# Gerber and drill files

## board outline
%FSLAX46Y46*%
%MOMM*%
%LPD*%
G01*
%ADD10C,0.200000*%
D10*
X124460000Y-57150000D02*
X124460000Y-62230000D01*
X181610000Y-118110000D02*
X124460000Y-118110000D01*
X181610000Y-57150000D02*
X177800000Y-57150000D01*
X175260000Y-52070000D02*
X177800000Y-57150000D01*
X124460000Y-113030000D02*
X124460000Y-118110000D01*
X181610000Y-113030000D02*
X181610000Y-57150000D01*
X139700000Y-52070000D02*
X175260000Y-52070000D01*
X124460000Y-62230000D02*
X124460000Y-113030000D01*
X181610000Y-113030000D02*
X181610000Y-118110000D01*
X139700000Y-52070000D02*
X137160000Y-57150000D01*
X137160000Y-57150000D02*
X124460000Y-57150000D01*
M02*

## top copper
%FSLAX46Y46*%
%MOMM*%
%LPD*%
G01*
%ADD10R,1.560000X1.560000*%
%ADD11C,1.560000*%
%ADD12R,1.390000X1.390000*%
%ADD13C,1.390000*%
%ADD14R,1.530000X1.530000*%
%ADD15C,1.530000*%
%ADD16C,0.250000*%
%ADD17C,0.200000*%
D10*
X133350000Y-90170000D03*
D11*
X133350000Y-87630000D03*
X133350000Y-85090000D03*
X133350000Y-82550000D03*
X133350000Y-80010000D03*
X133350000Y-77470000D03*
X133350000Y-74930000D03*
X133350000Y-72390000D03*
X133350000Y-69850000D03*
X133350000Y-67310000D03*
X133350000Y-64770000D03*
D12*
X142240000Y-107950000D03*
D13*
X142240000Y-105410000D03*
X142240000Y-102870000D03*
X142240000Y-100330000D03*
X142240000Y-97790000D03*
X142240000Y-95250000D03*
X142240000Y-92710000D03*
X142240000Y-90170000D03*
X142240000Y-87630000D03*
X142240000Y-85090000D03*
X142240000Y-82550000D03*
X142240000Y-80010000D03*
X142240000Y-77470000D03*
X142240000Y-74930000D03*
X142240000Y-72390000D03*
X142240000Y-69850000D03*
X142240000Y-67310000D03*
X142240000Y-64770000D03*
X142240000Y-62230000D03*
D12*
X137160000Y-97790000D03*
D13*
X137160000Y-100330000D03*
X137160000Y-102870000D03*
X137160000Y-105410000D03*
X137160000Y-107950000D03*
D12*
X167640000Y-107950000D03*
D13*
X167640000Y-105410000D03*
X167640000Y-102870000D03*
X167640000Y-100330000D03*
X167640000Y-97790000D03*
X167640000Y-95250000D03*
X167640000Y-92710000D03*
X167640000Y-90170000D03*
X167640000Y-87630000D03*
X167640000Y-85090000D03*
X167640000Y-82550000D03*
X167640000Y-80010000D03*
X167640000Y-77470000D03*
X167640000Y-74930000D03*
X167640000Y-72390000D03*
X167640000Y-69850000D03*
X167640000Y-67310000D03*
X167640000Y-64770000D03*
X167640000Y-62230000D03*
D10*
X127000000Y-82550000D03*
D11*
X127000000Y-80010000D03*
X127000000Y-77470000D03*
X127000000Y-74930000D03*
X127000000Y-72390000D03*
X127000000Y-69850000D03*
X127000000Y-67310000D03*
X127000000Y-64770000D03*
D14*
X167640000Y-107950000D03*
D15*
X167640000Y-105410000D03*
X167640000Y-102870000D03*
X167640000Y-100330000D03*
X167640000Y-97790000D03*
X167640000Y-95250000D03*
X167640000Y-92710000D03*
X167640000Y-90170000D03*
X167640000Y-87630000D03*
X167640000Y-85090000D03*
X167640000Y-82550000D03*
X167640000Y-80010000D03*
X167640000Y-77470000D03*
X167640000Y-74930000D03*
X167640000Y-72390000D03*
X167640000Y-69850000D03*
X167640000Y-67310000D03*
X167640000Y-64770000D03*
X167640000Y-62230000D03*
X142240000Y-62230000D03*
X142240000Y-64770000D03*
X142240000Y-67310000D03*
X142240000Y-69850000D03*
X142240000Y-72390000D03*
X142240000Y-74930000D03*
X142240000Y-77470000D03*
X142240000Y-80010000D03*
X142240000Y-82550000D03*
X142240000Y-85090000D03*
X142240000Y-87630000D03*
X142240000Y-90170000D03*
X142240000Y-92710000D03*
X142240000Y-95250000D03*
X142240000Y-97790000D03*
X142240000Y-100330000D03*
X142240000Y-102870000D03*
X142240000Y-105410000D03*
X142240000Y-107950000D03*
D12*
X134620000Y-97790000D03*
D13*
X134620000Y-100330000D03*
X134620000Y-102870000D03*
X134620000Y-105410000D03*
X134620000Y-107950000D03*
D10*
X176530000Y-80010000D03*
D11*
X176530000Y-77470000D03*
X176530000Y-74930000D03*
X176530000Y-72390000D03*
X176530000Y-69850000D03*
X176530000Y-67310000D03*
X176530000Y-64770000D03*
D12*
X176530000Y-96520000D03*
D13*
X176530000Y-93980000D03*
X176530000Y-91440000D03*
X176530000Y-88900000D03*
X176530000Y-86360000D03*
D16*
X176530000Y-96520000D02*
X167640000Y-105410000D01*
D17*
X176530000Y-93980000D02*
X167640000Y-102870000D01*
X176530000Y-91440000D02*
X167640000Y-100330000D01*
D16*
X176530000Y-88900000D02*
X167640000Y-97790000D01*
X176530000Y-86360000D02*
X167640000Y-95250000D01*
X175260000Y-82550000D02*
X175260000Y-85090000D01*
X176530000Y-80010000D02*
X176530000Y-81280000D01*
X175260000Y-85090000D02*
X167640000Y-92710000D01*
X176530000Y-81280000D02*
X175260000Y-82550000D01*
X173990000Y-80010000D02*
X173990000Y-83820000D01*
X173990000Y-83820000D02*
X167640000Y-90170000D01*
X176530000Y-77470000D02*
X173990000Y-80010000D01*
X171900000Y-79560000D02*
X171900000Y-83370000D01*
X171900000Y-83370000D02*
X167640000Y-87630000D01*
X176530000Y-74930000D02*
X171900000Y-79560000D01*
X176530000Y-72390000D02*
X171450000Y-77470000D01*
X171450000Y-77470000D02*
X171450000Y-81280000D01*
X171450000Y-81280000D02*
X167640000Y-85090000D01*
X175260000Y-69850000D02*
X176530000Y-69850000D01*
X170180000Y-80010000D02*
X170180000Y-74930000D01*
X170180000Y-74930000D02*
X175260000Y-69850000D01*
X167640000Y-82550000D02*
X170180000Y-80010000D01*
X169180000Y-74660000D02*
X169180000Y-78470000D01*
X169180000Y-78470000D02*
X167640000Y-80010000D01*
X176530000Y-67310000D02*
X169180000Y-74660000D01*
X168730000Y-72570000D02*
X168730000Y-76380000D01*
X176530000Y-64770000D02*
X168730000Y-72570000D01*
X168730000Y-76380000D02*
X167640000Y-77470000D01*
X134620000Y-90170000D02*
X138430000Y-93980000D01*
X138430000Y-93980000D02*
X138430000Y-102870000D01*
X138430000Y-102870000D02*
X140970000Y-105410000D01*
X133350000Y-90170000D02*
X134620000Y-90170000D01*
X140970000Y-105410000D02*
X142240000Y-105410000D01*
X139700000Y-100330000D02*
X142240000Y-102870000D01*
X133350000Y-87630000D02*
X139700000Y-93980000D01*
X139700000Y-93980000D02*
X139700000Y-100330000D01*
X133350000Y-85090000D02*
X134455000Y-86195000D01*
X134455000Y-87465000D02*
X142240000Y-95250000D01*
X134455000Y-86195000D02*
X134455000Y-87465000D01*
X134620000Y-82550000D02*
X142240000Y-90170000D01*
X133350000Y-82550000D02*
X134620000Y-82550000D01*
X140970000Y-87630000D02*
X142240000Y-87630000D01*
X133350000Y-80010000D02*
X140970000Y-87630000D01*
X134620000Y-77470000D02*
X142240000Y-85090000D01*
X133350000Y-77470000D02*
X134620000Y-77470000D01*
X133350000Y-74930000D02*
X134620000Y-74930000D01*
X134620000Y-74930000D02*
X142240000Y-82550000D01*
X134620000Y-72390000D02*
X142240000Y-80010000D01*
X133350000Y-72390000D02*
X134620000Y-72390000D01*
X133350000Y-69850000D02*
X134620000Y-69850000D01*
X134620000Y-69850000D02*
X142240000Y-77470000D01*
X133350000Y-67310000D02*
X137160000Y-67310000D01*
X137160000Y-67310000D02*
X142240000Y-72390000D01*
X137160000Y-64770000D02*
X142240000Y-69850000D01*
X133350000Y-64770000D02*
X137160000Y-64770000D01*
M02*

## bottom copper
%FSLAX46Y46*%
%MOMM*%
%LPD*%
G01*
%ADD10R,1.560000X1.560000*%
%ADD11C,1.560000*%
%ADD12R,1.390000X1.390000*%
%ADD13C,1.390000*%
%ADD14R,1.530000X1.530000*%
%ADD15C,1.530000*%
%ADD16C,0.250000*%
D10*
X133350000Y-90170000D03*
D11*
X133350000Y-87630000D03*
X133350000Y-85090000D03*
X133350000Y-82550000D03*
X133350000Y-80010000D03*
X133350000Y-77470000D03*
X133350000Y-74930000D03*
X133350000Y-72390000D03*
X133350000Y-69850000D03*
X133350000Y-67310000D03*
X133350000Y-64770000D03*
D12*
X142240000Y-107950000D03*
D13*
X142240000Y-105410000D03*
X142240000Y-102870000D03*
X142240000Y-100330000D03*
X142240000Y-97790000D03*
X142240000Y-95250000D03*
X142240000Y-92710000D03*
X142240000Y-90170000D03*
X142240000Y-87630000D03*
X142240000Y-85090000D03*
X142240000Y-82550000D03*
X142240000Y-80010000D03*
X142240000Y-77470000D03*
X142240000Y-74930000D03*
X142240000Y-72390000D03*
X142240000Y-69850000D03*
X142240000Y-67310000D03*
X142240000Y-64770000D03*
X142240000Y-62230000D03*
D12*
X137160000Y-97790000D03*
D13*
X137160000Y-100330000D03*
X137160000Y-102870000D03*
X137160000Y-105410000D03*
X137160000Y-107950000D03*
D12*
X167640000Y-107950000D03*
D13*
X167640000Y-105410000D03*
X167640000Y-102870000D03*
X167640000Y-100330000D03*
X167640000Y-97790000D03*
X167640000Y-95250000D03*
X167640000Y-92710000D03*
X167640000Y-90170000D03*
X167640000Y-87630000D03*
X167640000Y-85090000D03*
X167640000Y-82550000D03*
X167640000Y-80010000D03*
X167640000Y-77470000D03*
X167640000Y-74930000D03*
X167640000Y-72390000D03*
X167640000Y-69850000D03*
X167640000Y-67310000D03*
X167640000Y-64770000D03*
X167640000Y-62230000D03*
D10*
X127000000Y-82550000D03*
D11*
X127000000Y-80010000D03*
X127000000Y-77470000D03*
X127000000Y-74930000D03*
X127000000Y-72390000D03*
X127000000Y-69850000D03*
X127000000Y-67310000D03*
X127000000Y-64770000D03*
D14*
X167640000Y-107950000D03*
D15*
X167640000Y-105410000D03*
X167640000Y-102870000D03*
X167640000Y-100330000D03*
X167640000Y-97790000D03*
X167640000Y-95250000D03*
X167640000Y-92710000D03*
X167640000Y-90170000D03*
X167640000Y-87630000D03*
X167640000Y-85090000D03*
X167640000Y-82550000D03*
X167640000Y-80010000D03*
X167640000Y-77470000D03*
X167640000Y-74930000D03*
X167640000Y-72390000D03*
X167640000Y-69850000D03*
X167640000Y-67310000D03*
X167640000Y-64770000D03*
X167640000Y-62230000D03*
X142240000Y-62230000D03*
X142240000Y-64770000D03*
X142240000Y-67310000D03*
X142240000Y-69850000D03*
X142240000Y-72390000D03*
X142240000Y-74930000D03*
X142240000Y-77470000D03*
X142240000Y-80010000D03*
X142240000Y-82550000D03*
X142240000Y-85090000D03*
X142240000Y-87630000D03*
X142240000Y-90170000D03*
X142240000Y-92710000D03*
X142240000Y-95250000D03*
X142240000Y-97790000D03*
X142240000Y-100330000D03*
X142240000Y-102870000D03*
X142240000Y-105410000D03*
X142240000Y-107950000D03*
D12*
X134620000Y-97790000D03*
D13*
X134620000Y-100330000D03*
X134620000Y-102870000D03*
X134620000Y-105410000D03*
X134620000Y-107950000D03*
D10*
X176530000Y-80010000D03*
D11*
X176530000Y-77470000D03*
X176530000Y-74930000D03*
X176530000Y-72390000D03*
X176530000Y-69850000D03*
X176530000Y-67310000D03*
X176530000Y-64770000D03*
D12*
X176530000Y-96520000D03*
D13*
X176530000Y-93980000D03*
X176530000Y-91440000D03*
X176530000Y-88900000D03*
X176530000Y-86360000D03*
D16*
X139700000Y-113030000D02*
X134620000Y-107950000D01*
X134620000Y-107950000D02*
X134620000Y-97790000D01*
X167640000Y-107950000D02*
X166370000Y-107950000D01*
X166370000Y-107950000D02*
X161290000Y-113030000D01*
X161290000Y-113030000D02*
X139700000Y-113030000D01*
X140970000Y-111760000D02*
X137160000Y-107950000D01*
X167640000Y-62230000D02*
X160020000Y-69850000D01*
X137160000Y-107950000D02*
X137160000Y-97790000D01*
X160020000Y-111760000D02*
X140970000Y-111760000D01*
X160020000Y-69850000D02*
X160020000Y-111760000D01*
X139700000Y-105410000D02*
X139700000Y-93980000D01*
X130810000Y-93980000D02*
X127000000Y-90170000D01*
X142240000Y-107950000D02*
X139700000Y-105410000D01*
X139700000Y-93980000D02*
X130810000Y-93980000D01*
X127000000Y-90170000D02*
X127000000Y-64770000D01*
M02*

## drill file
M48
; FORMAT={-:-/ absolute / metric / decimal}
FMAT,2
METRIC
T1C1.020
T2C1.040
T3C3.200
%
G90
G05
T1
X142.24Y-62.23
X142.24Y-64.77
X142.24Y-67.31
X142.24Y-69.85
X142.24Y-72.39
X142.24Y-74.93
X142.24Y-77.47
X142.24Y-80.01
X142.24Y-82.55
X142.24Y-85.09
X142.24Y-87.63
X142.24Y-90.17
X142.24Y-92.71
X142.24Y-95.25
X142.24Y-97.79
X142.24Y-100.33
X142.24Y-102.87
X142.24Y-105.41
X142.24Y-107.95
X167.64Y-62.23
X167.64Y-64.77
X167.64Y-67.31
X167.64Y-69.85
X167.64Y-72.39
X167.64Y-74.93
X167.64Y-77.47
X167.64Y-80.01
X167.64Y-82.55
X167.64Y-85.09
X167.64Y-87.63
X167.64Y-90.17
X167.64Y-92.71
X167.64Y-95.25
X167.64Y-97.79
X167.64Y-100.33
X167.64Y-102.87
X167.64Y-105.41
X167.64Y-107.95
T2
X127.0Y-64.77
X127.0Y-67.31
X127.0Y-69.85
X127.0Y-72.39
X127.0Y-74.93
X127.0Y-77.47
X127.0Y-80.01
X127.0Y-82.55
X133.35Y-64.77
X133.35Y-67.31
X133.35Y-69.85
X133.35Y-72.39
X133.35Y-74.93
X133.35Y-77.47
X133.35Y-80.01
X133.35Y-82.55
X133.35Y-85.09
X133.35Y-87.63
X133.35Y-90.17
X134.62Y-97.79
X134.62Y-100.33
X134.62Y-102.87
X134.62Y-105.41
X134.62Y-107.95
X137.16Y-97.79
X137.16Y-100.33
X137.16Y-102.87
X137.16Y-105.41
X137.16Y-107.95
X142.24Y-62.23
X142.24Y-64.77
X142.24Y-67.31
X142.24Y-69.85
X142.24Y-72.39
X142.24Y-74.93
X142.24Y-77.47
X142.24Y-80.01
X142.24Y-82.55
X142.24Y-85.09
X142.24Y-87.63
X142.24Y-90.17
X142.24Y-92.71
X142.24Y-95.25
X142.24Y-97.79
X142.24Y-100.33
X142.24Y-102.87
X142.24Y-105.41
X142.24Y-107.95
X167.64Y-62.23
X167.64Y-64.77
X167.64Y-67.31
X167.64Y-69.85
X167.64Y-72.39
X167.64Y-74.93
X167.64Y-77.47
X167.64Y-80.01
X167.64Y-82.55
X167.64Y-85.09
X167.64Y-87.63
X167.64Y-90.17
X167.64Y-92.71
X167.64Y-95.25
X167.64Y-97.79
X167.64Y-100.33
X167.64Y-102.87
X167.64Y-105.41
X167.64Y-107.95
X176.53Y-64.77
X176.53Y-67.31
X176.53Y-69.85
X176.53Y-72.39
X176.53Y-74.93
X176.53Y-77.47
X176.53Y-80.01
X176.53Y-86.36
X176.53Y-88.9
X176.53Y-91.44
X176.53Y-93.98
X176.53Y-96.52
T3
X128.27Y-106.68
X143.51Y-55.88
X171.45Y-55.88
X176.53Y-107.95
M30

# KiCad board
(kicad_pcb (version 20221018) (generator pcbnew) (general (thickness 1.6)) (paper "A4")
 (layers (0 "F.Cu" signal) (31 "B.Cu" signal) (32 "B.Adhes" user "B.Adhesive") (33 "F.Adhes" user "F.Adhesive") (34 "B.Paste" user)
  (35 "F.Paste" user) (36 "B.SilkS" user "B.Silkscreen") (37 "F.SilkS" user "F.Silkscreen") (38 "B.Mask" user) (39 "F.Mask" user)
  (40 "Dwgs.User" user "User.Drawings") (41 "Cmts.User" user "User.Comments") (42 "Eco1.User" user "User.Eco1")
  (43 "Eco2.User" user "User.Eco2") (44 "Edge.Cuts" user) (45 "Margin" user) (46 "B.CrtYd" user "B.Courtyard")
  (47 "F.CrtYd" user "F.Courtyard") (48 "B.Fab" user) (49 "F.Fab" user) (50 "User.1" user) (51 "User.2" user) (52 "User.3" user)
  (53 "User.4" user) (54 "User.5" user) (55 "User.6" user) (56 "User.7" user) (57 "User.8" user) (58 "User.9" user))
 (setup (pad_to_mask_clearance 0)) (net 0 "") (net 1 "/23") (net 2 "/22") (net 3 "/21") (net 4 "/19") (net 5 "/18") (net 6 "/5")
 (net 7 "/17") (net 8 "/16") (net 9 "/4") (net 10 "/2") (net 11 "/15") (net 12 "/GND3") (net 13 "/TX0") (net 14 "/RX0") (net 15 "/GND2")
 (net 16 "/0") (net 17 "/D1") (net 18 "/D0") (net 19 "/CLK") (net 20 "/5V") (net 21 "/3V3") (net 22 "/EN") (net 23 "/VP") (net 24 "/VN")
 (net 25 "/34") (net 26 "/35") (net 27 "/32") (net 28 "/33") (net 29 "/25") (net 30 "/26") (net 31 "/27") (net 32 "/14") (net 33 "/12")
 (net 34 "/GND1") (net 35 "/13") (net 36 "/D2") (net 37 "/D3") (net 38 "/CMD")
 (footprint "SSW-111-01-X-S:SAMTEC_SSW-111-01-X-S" (layer "F.Cu") (at 133.35 77.47 90)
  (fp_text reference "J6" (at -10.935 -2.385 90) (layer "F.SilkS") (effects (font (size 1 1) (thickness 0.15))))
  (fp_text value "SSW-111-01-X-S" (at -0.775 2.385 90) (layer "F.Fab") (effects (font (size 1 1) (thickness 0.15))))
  (pad "01" thru_hole rect (at -12.7 0 90) (size 1.56 1.56) (drill 1.04) (layers "*.Cu" "*.Mask") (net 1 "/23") (solder_mask_margin 0.102))
  (pad "02" thru_hole circle (at -10.16 0 90) (size 1.56 1.56) (drill 1.04) (layers "*.Cu" "*.Mask") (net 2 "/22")
   (solder_mask_margin 0.102))
  (pad "03" thru_hole circle (at -7.62 0 90) (size 1.56 1.56) (drill 1.04) (layers "*.Cu" "*.Mask") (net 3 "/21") (solder_mask_margin 0.102))
  (pad "04" thru_hole circle (at -5.08 0 90) (size 1.56 1.56) (drill 1.04) (layers "*.Cu" "*.Mask") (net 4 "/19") (solder_mask_margin 0.102))
  (pad "05" thru_hole circle (at -2.54 0 90) (size 1.56 1.56) (drill 1.04) (layers "*.Cu" "*.Mask") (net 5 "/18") (solder_mask_margin 0.102))
  (pad "06" thru_hole circle (at 0 0 90) (size 1.56 1.56) (drill 1.04) (layers "*.Cu" "*.Mask") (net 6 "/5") (solder_mask_margin 0.102))
  (pad "07" thru_hole circle (at 2.54 0 90) (size 1.56 1.56) (drill 1.04) (layers "*.Cu" "*.Mask") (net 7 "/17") (solder_mask_margin 0.102))
  (pad "08" thru_hole circle (at 5.08 0 90) (size 1.56 1.56) (drill 1.04) (layers "*.Cu" "*.Mask") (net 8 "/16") (solder_mask_margin 0.102))
  (pad "09" thru_hole circle (at 7.62 0 90) (size 1.56 1.56) (drill 1.04) (layers "*.Cu" "*.Mask") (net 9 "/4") (solder_mask_margin 0.102))
  (pad "10" thru_hole circle (at 10.16 0 90) (size 1.56 1.56) (drill 1.04) (layers "*.Cu" "*.Mask") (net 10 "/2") (solder_mask_margin 0.102))
  (pad "11" thru_hole circle (at 12.7 0 90) (size 1.56 1.56) (drill 1.04) (layers "*.Cu" "*.Mask") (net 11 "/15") (solder_mask_margin 0.102)))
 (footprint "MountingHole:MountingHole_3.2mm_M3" (layer "F.Cu") (at 128.27 106.68 180)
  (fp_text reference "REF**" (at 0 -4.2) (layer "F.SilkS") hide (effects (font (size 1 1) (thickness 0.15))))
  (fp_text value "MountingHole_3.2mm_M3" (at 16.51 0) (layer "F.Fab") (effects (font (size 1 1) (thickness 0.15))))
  (pad "" np_thru_hole circle (at 0 0 180) (size 3.2 3.2) (drill 3.2) (layers "F&B.Cu" "*.Mask")))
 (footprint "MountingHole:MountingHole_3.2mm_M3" (layer "F.Cu") (at 143.51 55.88 180)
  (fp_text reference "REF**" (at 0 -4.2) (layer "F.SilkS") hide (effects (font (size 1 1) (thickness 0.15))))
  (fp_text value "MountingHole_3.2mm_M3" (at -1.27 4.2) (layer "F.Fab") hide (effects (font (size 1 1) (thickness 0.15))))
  (pad "" np_thru_hole circle (at 0 0 180) (size 3.2 3.2) (drill 3.2) (layers "F&B.Cu" "*.Mask")))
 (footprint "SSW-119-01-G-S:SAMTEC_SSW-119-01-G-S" (layer "F.Cu") (at 142.24 107.95 90)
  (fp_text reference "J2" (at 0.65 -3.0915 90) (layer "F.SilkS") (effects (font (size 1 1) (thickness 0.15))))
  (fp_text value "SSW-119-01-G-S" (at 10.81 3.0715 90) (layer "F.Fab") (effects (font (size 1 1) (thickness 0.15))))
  (pad "01" thru_hole rect (at 0 0 90) (size 1.39 1.39) (drill 1.04) (layers "*.Cu" "*.Mask") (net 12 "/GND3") (solder_mask_margin 0.102))
  (pad "02" thru_hole circle (at 2.54 0 90) (size 1.39 1.39) (drill 1.04) (layers "*.Cu" "*.Mask") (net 1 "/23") (solder_mask_margin 0.102))
  (pad "03" thru_hole circle (at 5.08 0 90) (size 1.39 1.39) (drill 1.04) (layers "*.Cu" "*.Mask") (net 2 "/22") (solder_mask_margin 0.102))
  (pad "04" thru_hole circle (at 7.62 0 90) (size 1.39 1.39) (drill 1.04) (layers "*.Cu" "*.Mask") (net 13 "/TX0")
   (solder_mask_margin 0.102))
  (pad "05" thru_hole circle (at 10.16 0 90) (size 1.39 1.39) (drill 1.04) (layers "*.Cu" "*.Mask") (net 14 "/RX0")
   (solder_mask_margin 0.102))
  (pad "06" thru_hole circle (at 12.7 0 90) (size 1.39 1.39) (drill 1.04) (layers "*.Cu" "*.Mask") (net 3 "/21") (solder_mask_margin 0.102))
  (pad "07" thru_hole circle (at 15.24 0 90) (size 1.39 1.39) (drill 1.04) (layers "*.Cu" "*.Mask") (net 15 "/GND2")
   (solder_mask_margin 0.102))
  (pad "08" thru_hole circle (at 17.78 0 90) (size 1.39 1.39) (drill 1.04) (layers "*.Cu" "*.Mask") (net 4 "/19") (solder_mask_margin 0.102))
  (pad "09" thru_hole circle (at 20.32 0 90) (size 1.39 1.39) (drill 1.04) (layers "*.Cu" "*.Mask") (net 5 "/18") (solder_mask_margin 0.102))
  (pad "10" thru_hole circle (at 22.86 0 90) (size 1.39 1.39) (drill 1.04) (layers "*.Cu" "*.Mask") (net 6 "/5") (solder_mask_margin 0.102))
  (pad "11" thru_hole circle (at 25.4 0 90) (size 1.39 1.39) (drill 1.04) (layers "*.Cu" "*.Mask") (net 7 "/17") (solder_mask_margin 0.102))
  (pad "12" thru_hole circle (at 27.94 0 90) (size 1.39 1.39) (drill 1.04) (layers "*.Cu" "*.Mask") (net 8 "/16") (solder_mask_margin 0.102))
  (pad "13" thru_hole circle (at 30.48 0 90) (size 1.39 1.39) (drill 1.04) (layers "*.Cu" "*.Mask") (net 9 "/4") (solder_mask_margin 0.102))
  (pad "14" thru_hole circle (at 33.02 0 90) (size 1.39 1.39) (drill 1.04) (layers "*.Cu" "*.Mask") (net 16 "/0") (solder_mask_margin 0.102))
  (pad "15" thru_hole circle (at 35.56 0 90) (size 1.39 1.39) (drill 1.04) (layers "*.Cu" "*.Mask") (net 10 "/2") (solder_mask_margin 0.102))
  (pad "16" thru_hole circle (at 38.1 0 90) (size 1.39 1.39) (drill 1.04) (layers "*.Cu" "*.Mask") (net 11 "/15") (solder_mask_margin 0.102))
  (pad "17" thru_hole circle (at 40.64 0 90) (size 1.39 1.39) (drill 1.04) (layers "*.Cu" "*.Mask") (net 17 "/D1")
   (solder_mask_margin 0.102))
  (pad "18" thru_hole circle (at 43.18 0 90) (size 1.39 1.39) (drill 1.04) (layers "*.Cu" "*.Mask") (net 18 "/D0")
   (solder_mask_margin 0.102))
  (pad "19" thru_hole circle (at 45.72 0 90) (size 1.39 1.39) (drill 1.04) (layers "*.Cu" "*.Mask") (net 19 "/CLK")
   (solder_mask_margin 0.102)))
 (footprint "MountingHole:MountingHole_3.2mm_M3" (layer "F.Cu") (at 171.45 55.88 180)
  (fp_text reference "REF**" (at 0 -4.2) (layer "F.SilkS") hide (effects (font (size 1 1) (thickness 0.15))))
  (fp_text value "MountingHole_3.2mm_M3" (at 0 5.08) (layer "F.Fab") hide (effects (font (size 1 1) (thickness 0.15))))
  (pad "" np_thru_hole circle (at 0 0 180) (size 3.2 3.2) (drill 3.2) (layers "F&B.Cu" "*.Mask")))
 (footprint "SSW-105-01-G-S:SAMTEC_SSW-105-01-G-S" (layer "F.Cu") (at 137.16 97.79 -90)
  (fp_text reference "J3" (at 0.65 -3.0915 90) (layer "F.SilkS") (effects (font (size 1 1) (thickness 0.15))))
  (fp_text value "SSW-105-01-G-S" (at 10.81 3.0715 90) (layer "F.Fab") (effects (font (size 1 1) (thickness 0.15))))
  (pad "01" thru_hole rect (at 0 0 270) (size 1.39 1.39) (drill 1.04) (layers "*.Cu" "*.Mask") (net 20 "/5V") (solder_mask_margin 0.102))
  (pad "02" thru_hole circle (at 2.54 0 270) (size 1.39 1.39) (drill 1.04) (layers "*.Cu" "*.Mask") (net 20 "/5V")
   (solder_mask_margin 0.102))
  (pad "03" thru_hole circle (at 5.08 0 270) (size 1.39 1.39) (drill 1.04) (layers "*.Cu" "*.Mask") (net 20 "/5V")
   (solder_mask_margin 0.102))
  (pad "04" thru_hole circle (at 7.62 0 270) (size 1.39 1.39) (drill 1.04) (layers "*.Cu" "*.Mask") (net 20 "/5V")
   (solder_mask_margin 0.102))
  (pad "05" thru_hole circle (at 10.16 0 270) (size 1.39 1.39) (drill 1.04) (layers "*.Cu" "*.Mask") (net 20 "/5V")
   (solder_mask_margin 0.102)))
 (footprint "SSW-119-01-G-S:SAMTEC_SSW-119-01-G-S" (layer "F.Cu") (at 167.64 107.95 90)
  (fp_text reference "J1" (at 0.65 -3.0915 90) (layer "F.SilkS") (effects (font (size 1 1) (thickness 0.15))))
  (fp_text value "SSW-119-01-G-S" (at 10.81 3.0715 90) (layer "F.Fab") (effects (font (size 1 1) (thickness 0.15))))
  (pad "01" thru_hole rect (at 0 0 90) (size 1.39 1.39) (drill 1.04) (layers "*.Cu" "*.Mask") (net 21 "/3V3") (solder_mask_margin 0.102))
  (pad "02" thru_hole circle (at 2.54 0 90) (size 1.39 1.39) (drill 1.04) (layers "*.Cu" "*.Mask") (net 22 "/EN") (solder_mask_margin 0.102))
  (pad "03" thru_hole circle (at 5.08 0 90) (size 1.39 1.39) (drill 1.04) (layers "*.Cu" "*.Mask") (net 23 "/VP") (solder_mask_margin 0.102))
  (pad "04" thru_hole circle (at 7.62 0 90) (size 1.39 1.39) (drill 1.04) (layers "*.Cu" "*.Mask") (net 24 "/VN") (solder_mask_margin 0.102))
  (pad "05" thru_hole circle (at 10.16 0 90) (size 1.39 1.39) (drill 1.04) (layers "*.Cu" "*.Mask") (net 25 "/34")
   (solder_mask_margin 0.102))
  (pad "06" thru_hole circle (at 12.7 0 90) (size 1.39 1.39) (drill 1.04) (layers "*.Cu" "*.Mask") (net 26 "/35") (solder_mask_margin 0.102))
  (pad "07" thru_hole circle (at 15.24 0 90) (size 1.39 1.39) (drill 1.04) (layers "*.Cu" "*.Mask") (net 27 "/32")
   (solder_mask_margin 0.102))
  (pad "08" thru_hole circle (at 17.78 0 90) (size 1.39 1.39) (drill 1.04) (layers "*.Cu" "*.Mask") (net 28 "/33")
   (solder_mask_margin 0.102))
  (pad "09" thru_hole circle (at 20.32 0 90) (size 1.39 1.39) (drill 1.04) (layers "*.Cu" "*.Mask") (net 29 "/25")
   (solder_mask_margin 0.102))
  (pad "10" thru_hole circle (at 22.86 0 90) (size 1.39 1.39) (drill 1.04) (layers "*.Cu" "*.Mask") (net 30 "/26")
   (solder_mask_margin 0.102))
  (pad "11" thru_hole circle (at 25.4 0 90) (size 1.39 1.39) (drill 1.04) (layers "*.Cu" "*.Mask") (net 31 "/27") (solder_mask_margin 0.102))
  (pad "12" thru_hole circle (at 27.94 0 90) (size 1.39 1.39) (drill 1.04) (layers "*.Cu" "*.Mask") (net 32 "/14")
   (solder_mask_margin 0.102))
  (pad "13" thru_hole circle (at 30.48 0 90) (size 1.39 1.39) (drill 1.04) (layers "*.Cu" "*.Mask") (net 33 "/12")
   (solder_mask_margin 0.102))
  (pad "14" thru_hole circle (at 33.02 0 90) (size 1.39 1.39) (drill 1.04) (layers "*.Cu" "*.Mask") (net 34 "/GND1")
   (solder_mask_margin 0.102))
  (pad "15" thru_hole circle (at 35.56 0 90) (size 1.39 1.39) (drill 1.04) (layers "*.Cu" "*.Mask") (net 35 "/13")
   (solder_mask_margin 0.102))
  (pad "16" thru_hole circle (at 38.1 0 90) (size 1.39 1.39) (drill 1.04) (layers "*.Cu" "*.Mask") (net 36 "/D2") (solder_mask_margin 0.102))
  (pad "17" thru_hole circle (at 40.64 0 90) (size 1.39 1.39) (drill 1.04) (layers "*.Cu" "*.Mask") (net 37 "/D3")
   (solder_mask_margin 0.102))
  (pad "18" thru_hole circle (at 43.18 0 90) (size 1.39 1.39) (drill 1.04) (layers "*.Cu" "*.Mask") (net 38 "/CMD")
   (solder_mask_margin 0.102))
  (pad "19" thru_hole circle (at 45.72 0 90) (size 1.39 1.39) (drill 1.04) (layers "*.Cu" "*.Mask") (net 20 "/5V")
   (solder_mask_margin 0.102)))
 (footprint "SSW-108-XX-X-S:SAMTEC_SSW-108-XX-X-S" (layer "F.Cu") (at 127 73.66 90)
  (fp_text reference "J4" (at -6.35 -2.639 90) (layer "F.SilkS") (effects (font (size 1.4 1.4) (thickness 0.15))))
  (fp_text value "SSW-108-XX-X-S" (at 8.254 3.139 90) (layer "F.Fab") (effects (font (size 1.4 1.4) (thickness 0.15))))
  (pad "01" thru_hole rect (at -8.89 0 90) (size 1.56 1.56) (drill 1.04) (layers "*.Cu" "*.Mask") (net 12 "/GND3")
   (solder_mask_margin 0.102))
  (pad "02" thru_hole circle (at -6.35 0 90) (size 1.56 1.56) (drill 1.04) (layers "*.Cu" "*.Mask") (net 12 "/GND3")
   (solder_mask_margin 0.102))
  (pad "03" thru_hole circle (at -3.81 0 90) (size 1.56 1.56) (drill 1.04) (layers "*.Cu" "*.Mask") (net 12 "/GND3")
   (solder_mask_margin 0.102))
  (pad "04" thru_hole circle (at -1.27 0 90) (size 1.56 1.56) (drill 1.04) (layers "*.Cu" "*.Mask") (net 12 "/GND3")
   (solder_mask_margin 0.102))
  (pad "05" thru_hole circle (at 1.27 0 90) (size 1.56 1.56) (drill 1.04) (layers "*.Cu" "*.Mask") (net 12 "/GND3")
   (solder_mask_margin 0.102))
  (pad "06" thru_hole circle (at 3.81 0 90) (size 1.56 1.56) (drill 1.04) (layers "*.Cu" "*.Mask") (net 12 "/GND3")
   (solder_mask_margin 0.102))
  (pad "07" thru_hole circle (at 6.35 0 90) (size 1.56 1.56) (drill 1.04) (layers "*.Cu" "*.Mask") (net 12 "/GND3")
   (solder_mask_margin 0.102))
  (pad "08" thru_hole circle (at 8.89 0 90) (size 1.56 1.56) (drill 1.04) (layers "*.Cu" "*.Mask") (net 12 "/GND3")
   (solder_mask_margin 0.102)))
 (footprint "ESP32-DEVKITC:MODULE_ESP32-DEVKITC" (layer "F.Cu") (at 154.94 85.1 180)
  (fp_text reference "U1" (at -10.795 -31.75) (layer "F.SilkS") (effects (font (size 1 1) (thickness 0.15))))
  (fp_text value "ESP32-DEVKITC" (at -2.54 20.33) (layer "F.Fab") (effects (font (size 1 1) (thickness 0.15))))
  (pad "1" thru_hole rect (at -12.7 -22.85 180) (size 1.53 1.53) (drill 1.02) (layers "*.Cu" "*.Mask") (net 21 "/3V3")
   (solder_mask_margin 0.102))
  (pad "2" thru_hole circle (at -12.7 -20.31 180) (size 1.53 1.53) (drill 1.02) (layers "*.Cu" "*.Mask") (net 22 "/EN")
   (solder_mask_margin 0.102))
  (pad "3" thru_hole circle (at -12.7 -17.77 180) (size 1.53 1.53) (drill 1.02) (layers "*.Cu" "*.Mask") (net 23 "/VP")
   (solder_mask_margin 0.102))
  (pad "4" thru_hole circle (at -12.7 -15.23 180) (size 1.53 1.53) (drill 1.02) (layers "*.Cu" "*.Mask") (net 24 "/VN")
   (solder_mask_margin 0.102))
  (pad "5" thru_hole circle (at -12.7 -12.69 180) (size 1.53 1.53) (drill 1.02) (layers "*.Cu" "*.Mask") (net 25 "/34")
   (solder_mask_margin 0.102))
  (pad "6" thru_hole circle (at -12.7 -10.15 180) (size 1.53 1.53) (drill 1.02) (layers "*.Cu" "*.Mask") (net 26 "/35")
   (solder_mask_margin 0.102))
  (pad "7" thru_hole circle (at -12.7 -7.61 180) (size 1.53 1.53) (drill 1.02) (layers "*.Cu" "*.Mask") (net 27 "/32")
   (solder_mask_margin 0.102))
  (pad "8" thru_hole circle (at -12.7 -5.07 180) (size 1.53 1.53) (drill 1.02) (layers "*.Cu" "*.Mask") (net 28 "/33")
   (solder_mask_margin 0.102))
  (pad "9" thru_hole circle (at -12.7 -2.53 180) (size 1.53 1.53) (drill 1.02) (layers "*.Cu" "*.Mask") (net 29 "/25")
   (solder_mask_margin 0.102))
  (pad "10" thru_hole circle (at -12.7 0.01 180) (size 1.53 1.53) (drill 1.02) (layers "*.Cu" "*.Mask") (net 30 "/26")
   (solder_mask_margin 0.102))
  (pad "11" thru_hole circle (at -12.7 2.55 180) (size 1.53 1.53) (drill 1.02) (layers "*.Cu" "*.Mask") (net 31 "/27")
   (solder_mask_margin 0.102))
  (pad "12" thru_hole circle (at -12.7 5.09 180) (size 1.53 1.53) (drill 1.02) (layers "*.Cu" "*.Mask") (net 32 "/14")
   (solder_mask_margin 0.102))
  (pad "13" thru_hole circle (at -12.7 7.63 180) (size 1.53 1.53) (drill 1.02) (layers "*.Cu" "*.Mask") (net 33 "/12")
   (solder_mask_margin 0.102))
  (pad "14" thru_hole circle (at -12.7 10.17 180) (size 1.53 1.53) (drill 1.02) (layers "*.Cu" "*.Mask") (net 34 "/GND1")
   (solder_mask_margin 0.102))
  (pad "15" thru_hole circle (at -12.7 12.71 180) (size 1.53 1.53) (drill 1.02) (layers "*.Cu" "*.Mask") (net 35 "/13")
   (solder_mask_margin 0.102))
  (pad "16" thru_hole circle (at -12.7 15.25 180) (size 1.53 1.53) (drill 1.02) (layers "*.Cu" "*.Mask") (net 36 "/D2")
   (solder_mask_margin 0.102))
  (pad "17" thru_hole circle (at -12.7 17.79 180) (size 1.53 1.53) (drill 1.02) (layers "*.Cu" "*.Mask") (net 37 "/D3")
   (solder_mask_margin 0.102))
  (pad "18" thru_hole circle (at -12.7 20.33 180) (size 1.53 1.53) (drill 1.02) (layers "*.Cu" "*.Mask") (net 38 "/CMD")
   (solder_mask_margin 0.102))
  (pad "19" thru_hole circle (at -12.7 22.87 180) (size 1.53 1.53) (drill 1.02) (layers "*.Cu" "*.Mask") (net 20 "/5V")
   (solder_mask_margin 0.102))
  (pad "20" thru_hole circle (at 12.7 22.87 180) (size 1.53 1.53) (drill 1.02) (layers "*.Cu" "*.Mask") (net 19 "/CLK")
   (solder_mask_margin 0.102))
  (pad "21" thru_hole circle (at 12.7 20.33 180) (size 1.53 1.53) (drill 1.02) (layers "*.Cu" "*.Mask") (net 18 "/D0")
   (solder_mask_margin 0.102))
  (pad "22" thru_hole circle (at 12.7 17.79 180) (size 1.53 1.53) (drill 1.02) (layers "*.Cu" "*.Mask") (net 17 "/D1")
   (solder_mask_margin 0.102))
  (pad "23" thru_hole circle (at 12.7 15.25 180) (size 1.53 1.53) (drill 1.02) (layers "*.Cu" "*.Mask") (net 11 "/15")
   (solder_mask_margin 0.102))
  (pad "24" thru_hole circle (at 12.7 12.71 180) (size 1.53 1.53) (drill 1.02) (layers "*.Cu" "*.Mask") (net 10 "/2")
   (solder_mask_margin 0.102))
  (pad "25" thru_hole circle (at 12.7 10.17 180) (size 1.53 1.53) (drill 1.02) (layers "*.Cu" "*.Mask") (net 16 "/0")
   (solder_mask_margin 0.102))
  (pad "26" thru_hole circle (at 12.7 7.63 180) (size 1.53 1.53) (drill 1.02) (layers "*.Cu" "*.Mask") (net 9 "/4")
   (solder_mask_margin 0.102))
  (pad "27" thru_hole circle (at 12.7 5.09 180) (size 1.53 1.53) (drill 1.02) (layers "*.Cu" "*.Mask") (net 8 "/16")
   (solder_mask_margin 0.102))
  (pad "28" thru_hole circle (at 12.7 2.55 180) (size 1.53 1.53) (drill 1.02) (layers "*.Cu" "*.Mask") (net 7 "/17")
   (solder_mask_margin 0.102))
  (pad "29" thru_hole circle (at 12.7 0.01 180) (size 1.53 1.53) (drill 1.02) (layers "*.Cu" "*.Mask") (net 6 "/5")
   (solder_mask_margin 0.102))
  (pad "30" thru_hole circle (at 12.7 -2.53 180) (size 1.53 1.53) (drill 1.02) (layers "*.Cu" "*.Mask") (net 5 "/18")
   (solder_mask_margin 0.102))
  (pad "31" thru_hole circle (at 12.7 -5.07 180) (size 1.53 1.53) (drill 1.02) (layers "*.Cu" "*.Mask") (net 4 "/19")
   (solder_mask_margin 0.102))
  (pad "32" thru_hole circle (at 12.7 -7.61 180) (size 1.53 1.53) (drill 1.02) (layers "*.Cu" "*.Mask") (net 15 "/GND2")
   (solder_mask_margin 0.102))
  (pad "33" thru_hole circle (at 12.7 -10.15 180) (size 1.53 1.53) (drill 1.02) (layers "*.Cu" "*.Mask") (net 3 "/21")
   (solder_mask_margin 0.102))
  (pad "34" thru_hole circle (at 12.7 -12.69 180) (size 1.53 1.53) (drill 1.02) (layers "*.Cu" "*.Mask") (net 14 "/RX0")
   (solder_mask_margin 0.102))
  (pad "35" thru_hole circle (at 12.7 -15.23 180) (size 1.53 1.53) (drill 1.02) (layers "*.Cu" "*.Mask") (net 13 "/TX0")
   (solder_mask_margin 0.102))
  (pad "36" thru_hole circle (at 12.7 -17.77 180) (size 1.53 1.53) (drill 1.02) (layers "*.Cu" "*.Mask") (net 2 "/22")
   (solder_mask_margin 0.102))
  (pad "37" thru_hole circle (at 12.7 -20.31 180) (size 1.53 1.53) (drill 1.02) (layers "*.Cu" "*.Mask") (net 1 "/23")
   (solder_mask_margin 0.102))
  (pad "38" thru_hole circle (at 12.7 -22.85 180) (size 1.53 1.53) (drill 1.02) (layers "*.Cu" "*.Mask") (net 12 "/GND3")
   (solder_mask_margin 0.102)))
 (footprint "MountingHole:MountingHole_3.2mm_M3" (layer "F.Cu") (at 176.53 107.95 180)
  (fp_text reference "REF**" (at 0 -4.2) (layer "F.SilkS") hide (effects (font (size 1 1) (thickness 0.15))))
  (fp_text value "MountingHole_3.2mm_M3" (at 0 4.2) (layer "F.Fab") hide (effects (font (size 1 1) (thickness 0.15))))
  (pad "" np_thru_hole circle (at 0 0 180) (size 3.2 3.2) (drill 3.2) (layers "F&B.Cu" "*.Mask")))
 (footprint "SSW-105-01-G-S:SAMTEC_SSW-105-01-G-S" (layer "F.Cu") (at 134.62 97.79 -90)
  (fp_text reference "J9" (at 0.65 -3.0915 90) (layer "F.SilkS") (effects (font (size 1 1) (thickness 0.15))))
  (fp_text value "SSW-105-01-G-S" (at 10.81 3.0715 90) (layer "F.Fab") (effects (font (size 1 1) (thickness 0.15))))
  (pad "01" thru_hole rect (at 0 0 270) (size 1.39 1.39) (drill 1.04) (layers "*.Cu" "*.Mask") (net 21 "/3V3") (solder_mask_margin 0.102))
  (pad "02" thru_hole circle (at 2.54 0 270) (size 1.39 1.39) (drill 1.04) (layers "*.Cu" "*.Mask") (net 21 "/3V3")
   (solder_mask_margin 0.102))
  (pad "03" thru_hole circle (at 5.08 0 270) (size 1.39 1.39) (drill 1.04) (layers "*.Cu" "*.Mask") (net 21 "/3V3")
   (solder_mask_margin 0.102))
  (pad "04" thru_hole circle (at 7.62 0 270) (size 1.39 1.39) (drill 1.04) (layers "*.Cu" "*.Mask") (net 21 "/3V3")
   (solder_mask_margin 0.102))
  (pad "05" thru_hole circle (at 10.16 0 270) (size 1.39 1.39) (drill 1.04) (layers "*.Cu" "*.Mask") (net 21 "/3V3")
   (solder_mask_margin 0.102)))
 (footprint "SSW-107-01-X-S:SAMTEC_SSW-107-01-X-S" (layer "F.Cu") (at 176.53 72.39 90)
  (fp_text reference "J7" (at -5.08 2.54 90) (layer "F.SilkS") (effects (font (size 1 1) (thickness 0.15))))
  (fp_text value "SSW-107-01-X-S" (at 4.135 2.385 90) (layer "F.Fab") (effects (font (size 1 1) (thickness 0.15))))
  (pad "01" thru_hole rect (at -7.62 0 90) (size 1.56 1.56) (drill 1.04) (layers "*.Cu" "*.Mask") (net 27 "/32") (solder_mask_margin 0.102))
  (pad "02" thru_hole circle (at -5.08 0 90) (size 1.56 1.56) (drill 1.04) (layers "*.Cu" "*.Mask") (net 28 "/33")
   (solder_mask_margin 0.102))
  (pad "03" thru_hole circle (at -2.54 0 90) (size 1.56 1.56) (drill 1.04) (layers "*.Cu" "*.Mask") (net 29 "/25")
   (solder_mask_margin 0.102))
  (pad "04" thru_hole circle (at 0 0 90) (size 1.56 1.56) (drill 1.04) (layers "*.Cu" "*.Mask") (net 30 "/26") (solder_mask_margin 0.102))
  (pad "05" thru_hole circle (at 2.54 0 90) (size 1.56 1.56) (drill 1.04) (layers "*.Cu" "*.Mask") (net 31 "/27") (solder_mask_margin 0.102))
  (pad "06" thru_hole circle (at 5.08 0 90) (size 1.56 1.56) (drill 1.04) (layers "*.Cu" "*.Mask") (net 32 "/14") (solder_mask_margin 0.102))
  (pad "07" thru_hole circle (at 7.62 0 90) (size 1.56 1.56) (drill 1.04) (layers "*.Cu" "*.Mask") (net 33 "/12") (solder_mask_margin 0.102)))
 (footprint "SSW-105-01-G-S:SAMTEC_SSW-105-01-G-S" (layer "F.Cu") (at 176.53 96.52 90)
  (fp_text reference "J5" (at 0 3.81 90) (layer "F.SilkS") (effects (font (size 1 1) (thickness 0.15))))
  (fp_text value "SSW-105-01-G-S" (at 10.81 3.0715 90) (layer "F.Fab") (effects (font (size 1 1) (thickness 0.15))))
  (pad "01" thru_hole rect (at 0 0 90) (size 1.39 1.39) (drill 1.04) (layers "*.Cu" "*.Mask") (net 22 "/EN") (solder_mask_margin 0.102))
  (pad "02" thru_hole circle (at 2.54 0 90) (size 1.39 1.39) (drill 1.04) (layers "*.Cu" "*.Mask") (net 23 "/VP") (solder_mask_margin 0.102))
  (pad "03" thru_hole circle (at 5.08 0 90) (size 1.39 1.39) (drill 1.04) (layers "*.Cu" "*.Mask") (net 24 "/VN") (solder_mask_margin 0.102))
  (pad "04" thru_hole circle (at 7.62 0 90) (size 1.39 1.39) (drill 1.04) (layers "*.Cu" "*.Mask") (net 25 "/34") (solder_mask_margin 0.102))
  (pad "05" thru_hole circle (at 10.16 0 90) (size 1.39 1.39) (drill 1.04) (layers "*.Cu" "*.Mask") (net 26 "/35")
   (solder_mask_margin 0.102)))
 (gr_line (start 124.46 57.15) (end 124.46 62.23) (stroke (width 0.2) (type default)) (layer "Edge.Cuts"))
 (gr_line (start 181.61 118.11) (end 124.46 118.11) (stroke (width 0.2) (type default)) (layer "Edge.Cuts"))
 (gr_line (start 181.61 57.15) (end 177.8 57.15) (stroke (width 0.2) (type default)) (layer "Edge.Cuts"))
 (gr_line (start 175.26 52.07) (end 177.8 57.15) (stroke (width 0.2) (type default)) (layer "Edge.Cuts"))
 (gr_line (start 124.46 113.03) (end 124.46 118.11) (stroke (width 0.2) (type default)) (layer "Edge.Cuts"))
 (gr_line (start 181.61 113.03) (end 181.61 57.15) (stroke (width 0.2) (type default)) (layer "Edge.Cuts"))
 (gr_line (start 139.7 52.07) (end 175.26 52.07) (stroke (width 0.2) (type default)) (layer "Edge.Cuts"))
 (gr_line (start 124.46 62.23) (end 124.46 113.03) (stroke (width 0.2) (type default)) (layer "Edge.Cuts"))
 (gr_line (start 181.61 113.03) (end 181.61 118.11) (stroke (width 0.2) (type default)) (layer "Edge.Cuts"))
 (gr_line (start 139.7 52.07) (end 137.16 57.15) (stroke (width 0.2) (type default)) (layer "Edge.Cuts"))
 (gr_line (start 137.16 57.15) (end 124.46 57.15) (stroke (width 0.2) (type default)) (layer "Edge.Cuts"))
 (segment (start 139.7 113.03) (end 134.62 107.95) (width 0.25) (layer "B.Cu") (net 21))
 (segment (start 134.62 107.95) (end 134.62 97.79) (width 0.25) (layer "B.Cu") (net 21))
 (segment (start 167.64 107.95) (end 166.37 107.95) (width 0.25) (layer "B.Cu") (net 21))
 (segment (start 166.37 107.95) (end 161.29 113.03) (width 0.25) (layer "B.Cu") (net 21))
 (segment (start 161.29 113.03) (end 139.7 113.03) (width 0.25) (layer "B.Cu") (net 21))
 (segment (start 176.53 96.52) (end 167.64 105.41) (width 0.25) (layer "F.Cu") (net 22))
 (segment (start 176.53 93.98) (end 167.64 102.87) (width 0.2) (layer "F.Cu") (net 23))
 (segment (start 176.53 91.44) (end 167.64 100.33) (width 0.2) (layer "F.Cu") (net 24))
 (segment (start 176.53 88.9) (end 167.64 97.79) (width 0.25) (layer "F.Cu") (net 25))
 (segment (start 176.53 86.36) (end 167.64 95.25) (width 0.25) (layer "F.Cu") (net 26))
 (segment (start 175.26 82.55) (end 175.26 85.09) (width 0.25) (layer "F.Cu") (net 27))
 (segment (start 176.53 80.01) (end 176.53 81.28) (width 0.25) (layer "F.Cu") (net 27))
 (segment (start 175.26 85.09) (end 167.64 92.71) (width 0.25) (layer "F.Cu") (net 27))
 (segment (start 176.53 81.28) (end 175.26 82.55) (width 0.25) (layer "F.Cu") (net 27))
 (segment (start 173.99 80.01) (end 173.99 83.82) (width 0.25) (layer "F.Cu") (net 28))
 (segment (start 173.99 83.82) (end 167.64 90.17) (width 0.25) (layer "F.Cu") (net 28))
 (segment (start 176.53 77.47) (end 173.99 80.01) (width 0.25) (layer "F.Cu") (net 28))
 (segment (start 171.9 79.56) (end 171.9 83.37) (width 0.25) (layer "F.Cu") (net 29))
 (segment (start 171.9 83.37) (end 167.64 87.63) (width 0.25) (layer "F.Cu") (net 29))
 (segment (start 176.53 74.93) (end 171.9 79.56) (width 0.25) (layer "F.Cu") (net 29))
 (segment (start 176.53 72.39) (end 171.45 77.47) (width 0.25) (layer "F.Cu") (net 30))
 (segment (start 171.45 77.47) (end 171.45 81.28) (width 0.25) (layer "F.Cu") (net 30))
 (segment (start 171.45 81.28) (end 167.64 85.09) (width 0.25) (layer "F.Cu") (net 30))
 (segment (start 175.26 69.85) (end 176.53 69.85) (width 0.25) (layer "F.Cu") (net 31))
 (segment (start 170.18 80.01) (end 170.18 74.93) (width 0.25) (layer "F.Cu") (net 31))
 (segment (start 170.18 74.93) (end 175.26 69.85) (width 0.25) (layer "F.Cu") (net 31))
 (segment (start 167.64 82.55) (end 170.18 80.01) (width 0.25) (layer "F.Cu") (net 31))
 (segment (start 169.18 74.66) (end 169.18 78.47) (width 0.25) (layer "F.Cu") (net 32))
 (segment (start 169.18 78.47) (end 167.64 80.01) (width 0.25) (layer "F.Cu") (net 32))
 (segment (start 176.53 67.31) (end 169.18 74.66) (width 0.25) (layer "F.Cu") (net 32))
 (segment (start 168.73 72.57) (end 168.73 76.38) (width 0.25) (layer "F.Cu") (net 33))
 (segment (start 176.53 64.77) (end 168.73 72.57) (width 0.25) (layer "F.Cu") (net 33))
 (segment (start 168.73 76.38) (end 167.64 77.47) (width 0.25) (layer "F.Cu") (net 33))
 (segment (start 140.97 111.76) (end 137.16 107.95) (width 0.25) (layer "B.Cu") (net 20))
 (segment (start 167.64 62.23) (end 160.02 69.85) (width 0.25) (layer "B.Cu") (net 20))
 (segment (start 137.16 107.95) (end 137.16 97.79) (width 0.25) (layer "B.Cu") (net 20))
 (segment (start 160.02 111.76) (end 140.97 111.76) (width 0.25) (layer "B.Cu") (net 20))
 (segment (start 160.02 69.85) (end 160.02 111.76) (width 0.25) (layer "B.Cu") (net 20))
 (segment (start 139.7 105.41) (end 139.7 93.98) (width 0.25) (layer "B.Cu") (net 12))
 (segment (start 130.81 93.98) (end 127 90.17) (width 0.25) (layer "B.Cu") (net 12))
 (segment (start 142.24 107.95) (end 139.7 105.41) (width 0.25) (layer "B.Cu") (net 12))
 (segment (start 139.7 93.98) (end 130.81 93.98) (width 0.25) (layer "B.Cu") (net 12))
 (segment (start 127 90.17) (end 127 64.77) (width 0.25) (layer "B.Cu") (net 12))
 (segment (start 134.62 90.17) (end 138.43 93.98) (width 0.25) (layer "F.Cu") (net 1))
 (segment (start 138.43 93.98) (end 138.43 102.87) (width 0.25) (layer "F.Cu") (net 1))
 (segment (start 138.43 102.87) (end 140.97 105.41) (width 0.25) (layer "F.Cu") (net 1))
 (segment (start 133.35 90.17) (end 134.62 90.17) (width 0.25) (layer "F.Cu") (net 1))
 (segment (start 140.97 105.41) (end 142.24 105.41) (width 0.25) (layer "F.Cu") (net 1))
 (segment (start 139.7 100.33) (end 142.24 102.87) (width 0.25) (layer "F.Cu") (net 2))
 (segment (start 133.35 87.63) (end 139.7 93.98) (width 0.25) (layer "F.Cu") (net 2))
 (segment (start 139.7 93.98) (end 139.7 100.33) (width 0.25) (layer "F.Cu") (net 2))
 (segment (start 133.35 85.09) (end 134.455 86.195) (width 0.25) (layer "F.Cu") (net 3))
 (segment (start 134.455 87.465) (end 142.24 95.25) (width 0.25) (layer "F.Cu") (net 3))
 (segment (start 134.455 86.195) (end 134.455 87.465) (width 0.25) (layer "F.Cu") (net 3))
 (segment (start 134.62 82.55) (end 142.24 90.17) (width 0.25) (layer "F.Cu") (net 4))
 (segment (start 133.35 82.55) (end 134.62 82.55) (width 0.25) (layer "F.Cu") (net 4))
 (segment (start 140.97 87.63) (end 142.24 87.63) (width 0.25) (layer "F.Cu") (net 5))
 (segment (start 133.35 80.01) (end 140.97 87.63) (width 0.25) (layer "F.Cu") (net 5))
 (segment (start 134.62 77.47) (end 142.24 85.09) (width 0.25) (layer "F.Cu") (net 6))
 (segment (start 133.35 77.47) (end 134.62 77.47) (width 0.25) (layer "F.Cu") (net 6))
 (segment (start 133.35 74.93) (end 134.62 74.93) (width 0.25) (layer "F.Cu") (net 7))
 (segment (start 134.62 74.93) (end 142.24 82.55) (width 0.25) (layer "F.Cu") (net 7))
 (segment (start 134.62 72.39) (end 142.24 80.01) (width 0.25) (layer "F.Cu") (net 8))
 (segment (start 133.35 72.39) (end 134.62 72.39) (width 0.25) (layer "F.Cu") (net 8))
 (segment (start 133.35 69.85) (end 134.62 69.85) (width 0.25) (layer "F.Cu") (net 9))
 (segment (start 134.62 69.85) (end 142.24 77.47) (width 0.25) (layer "F.Cu") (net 9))
 (segment (start 133.35 67.31) (end 137.16 67.31) (width 0.25) (layer "F.Cu") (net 10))
 (segment (start 137.16 67.31) (end 142.24 72.39) (width 0.25) (layer "F.Cu") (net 10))
 (segment (start 137.16 64.77) (end 142.24 69.85) (width 0.25) (layer "F.Cu") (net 11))
 (segment (start 133.35 64.77) (end 137.16 64.77) (width 0.25) (layer "F.Cu") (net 11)))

